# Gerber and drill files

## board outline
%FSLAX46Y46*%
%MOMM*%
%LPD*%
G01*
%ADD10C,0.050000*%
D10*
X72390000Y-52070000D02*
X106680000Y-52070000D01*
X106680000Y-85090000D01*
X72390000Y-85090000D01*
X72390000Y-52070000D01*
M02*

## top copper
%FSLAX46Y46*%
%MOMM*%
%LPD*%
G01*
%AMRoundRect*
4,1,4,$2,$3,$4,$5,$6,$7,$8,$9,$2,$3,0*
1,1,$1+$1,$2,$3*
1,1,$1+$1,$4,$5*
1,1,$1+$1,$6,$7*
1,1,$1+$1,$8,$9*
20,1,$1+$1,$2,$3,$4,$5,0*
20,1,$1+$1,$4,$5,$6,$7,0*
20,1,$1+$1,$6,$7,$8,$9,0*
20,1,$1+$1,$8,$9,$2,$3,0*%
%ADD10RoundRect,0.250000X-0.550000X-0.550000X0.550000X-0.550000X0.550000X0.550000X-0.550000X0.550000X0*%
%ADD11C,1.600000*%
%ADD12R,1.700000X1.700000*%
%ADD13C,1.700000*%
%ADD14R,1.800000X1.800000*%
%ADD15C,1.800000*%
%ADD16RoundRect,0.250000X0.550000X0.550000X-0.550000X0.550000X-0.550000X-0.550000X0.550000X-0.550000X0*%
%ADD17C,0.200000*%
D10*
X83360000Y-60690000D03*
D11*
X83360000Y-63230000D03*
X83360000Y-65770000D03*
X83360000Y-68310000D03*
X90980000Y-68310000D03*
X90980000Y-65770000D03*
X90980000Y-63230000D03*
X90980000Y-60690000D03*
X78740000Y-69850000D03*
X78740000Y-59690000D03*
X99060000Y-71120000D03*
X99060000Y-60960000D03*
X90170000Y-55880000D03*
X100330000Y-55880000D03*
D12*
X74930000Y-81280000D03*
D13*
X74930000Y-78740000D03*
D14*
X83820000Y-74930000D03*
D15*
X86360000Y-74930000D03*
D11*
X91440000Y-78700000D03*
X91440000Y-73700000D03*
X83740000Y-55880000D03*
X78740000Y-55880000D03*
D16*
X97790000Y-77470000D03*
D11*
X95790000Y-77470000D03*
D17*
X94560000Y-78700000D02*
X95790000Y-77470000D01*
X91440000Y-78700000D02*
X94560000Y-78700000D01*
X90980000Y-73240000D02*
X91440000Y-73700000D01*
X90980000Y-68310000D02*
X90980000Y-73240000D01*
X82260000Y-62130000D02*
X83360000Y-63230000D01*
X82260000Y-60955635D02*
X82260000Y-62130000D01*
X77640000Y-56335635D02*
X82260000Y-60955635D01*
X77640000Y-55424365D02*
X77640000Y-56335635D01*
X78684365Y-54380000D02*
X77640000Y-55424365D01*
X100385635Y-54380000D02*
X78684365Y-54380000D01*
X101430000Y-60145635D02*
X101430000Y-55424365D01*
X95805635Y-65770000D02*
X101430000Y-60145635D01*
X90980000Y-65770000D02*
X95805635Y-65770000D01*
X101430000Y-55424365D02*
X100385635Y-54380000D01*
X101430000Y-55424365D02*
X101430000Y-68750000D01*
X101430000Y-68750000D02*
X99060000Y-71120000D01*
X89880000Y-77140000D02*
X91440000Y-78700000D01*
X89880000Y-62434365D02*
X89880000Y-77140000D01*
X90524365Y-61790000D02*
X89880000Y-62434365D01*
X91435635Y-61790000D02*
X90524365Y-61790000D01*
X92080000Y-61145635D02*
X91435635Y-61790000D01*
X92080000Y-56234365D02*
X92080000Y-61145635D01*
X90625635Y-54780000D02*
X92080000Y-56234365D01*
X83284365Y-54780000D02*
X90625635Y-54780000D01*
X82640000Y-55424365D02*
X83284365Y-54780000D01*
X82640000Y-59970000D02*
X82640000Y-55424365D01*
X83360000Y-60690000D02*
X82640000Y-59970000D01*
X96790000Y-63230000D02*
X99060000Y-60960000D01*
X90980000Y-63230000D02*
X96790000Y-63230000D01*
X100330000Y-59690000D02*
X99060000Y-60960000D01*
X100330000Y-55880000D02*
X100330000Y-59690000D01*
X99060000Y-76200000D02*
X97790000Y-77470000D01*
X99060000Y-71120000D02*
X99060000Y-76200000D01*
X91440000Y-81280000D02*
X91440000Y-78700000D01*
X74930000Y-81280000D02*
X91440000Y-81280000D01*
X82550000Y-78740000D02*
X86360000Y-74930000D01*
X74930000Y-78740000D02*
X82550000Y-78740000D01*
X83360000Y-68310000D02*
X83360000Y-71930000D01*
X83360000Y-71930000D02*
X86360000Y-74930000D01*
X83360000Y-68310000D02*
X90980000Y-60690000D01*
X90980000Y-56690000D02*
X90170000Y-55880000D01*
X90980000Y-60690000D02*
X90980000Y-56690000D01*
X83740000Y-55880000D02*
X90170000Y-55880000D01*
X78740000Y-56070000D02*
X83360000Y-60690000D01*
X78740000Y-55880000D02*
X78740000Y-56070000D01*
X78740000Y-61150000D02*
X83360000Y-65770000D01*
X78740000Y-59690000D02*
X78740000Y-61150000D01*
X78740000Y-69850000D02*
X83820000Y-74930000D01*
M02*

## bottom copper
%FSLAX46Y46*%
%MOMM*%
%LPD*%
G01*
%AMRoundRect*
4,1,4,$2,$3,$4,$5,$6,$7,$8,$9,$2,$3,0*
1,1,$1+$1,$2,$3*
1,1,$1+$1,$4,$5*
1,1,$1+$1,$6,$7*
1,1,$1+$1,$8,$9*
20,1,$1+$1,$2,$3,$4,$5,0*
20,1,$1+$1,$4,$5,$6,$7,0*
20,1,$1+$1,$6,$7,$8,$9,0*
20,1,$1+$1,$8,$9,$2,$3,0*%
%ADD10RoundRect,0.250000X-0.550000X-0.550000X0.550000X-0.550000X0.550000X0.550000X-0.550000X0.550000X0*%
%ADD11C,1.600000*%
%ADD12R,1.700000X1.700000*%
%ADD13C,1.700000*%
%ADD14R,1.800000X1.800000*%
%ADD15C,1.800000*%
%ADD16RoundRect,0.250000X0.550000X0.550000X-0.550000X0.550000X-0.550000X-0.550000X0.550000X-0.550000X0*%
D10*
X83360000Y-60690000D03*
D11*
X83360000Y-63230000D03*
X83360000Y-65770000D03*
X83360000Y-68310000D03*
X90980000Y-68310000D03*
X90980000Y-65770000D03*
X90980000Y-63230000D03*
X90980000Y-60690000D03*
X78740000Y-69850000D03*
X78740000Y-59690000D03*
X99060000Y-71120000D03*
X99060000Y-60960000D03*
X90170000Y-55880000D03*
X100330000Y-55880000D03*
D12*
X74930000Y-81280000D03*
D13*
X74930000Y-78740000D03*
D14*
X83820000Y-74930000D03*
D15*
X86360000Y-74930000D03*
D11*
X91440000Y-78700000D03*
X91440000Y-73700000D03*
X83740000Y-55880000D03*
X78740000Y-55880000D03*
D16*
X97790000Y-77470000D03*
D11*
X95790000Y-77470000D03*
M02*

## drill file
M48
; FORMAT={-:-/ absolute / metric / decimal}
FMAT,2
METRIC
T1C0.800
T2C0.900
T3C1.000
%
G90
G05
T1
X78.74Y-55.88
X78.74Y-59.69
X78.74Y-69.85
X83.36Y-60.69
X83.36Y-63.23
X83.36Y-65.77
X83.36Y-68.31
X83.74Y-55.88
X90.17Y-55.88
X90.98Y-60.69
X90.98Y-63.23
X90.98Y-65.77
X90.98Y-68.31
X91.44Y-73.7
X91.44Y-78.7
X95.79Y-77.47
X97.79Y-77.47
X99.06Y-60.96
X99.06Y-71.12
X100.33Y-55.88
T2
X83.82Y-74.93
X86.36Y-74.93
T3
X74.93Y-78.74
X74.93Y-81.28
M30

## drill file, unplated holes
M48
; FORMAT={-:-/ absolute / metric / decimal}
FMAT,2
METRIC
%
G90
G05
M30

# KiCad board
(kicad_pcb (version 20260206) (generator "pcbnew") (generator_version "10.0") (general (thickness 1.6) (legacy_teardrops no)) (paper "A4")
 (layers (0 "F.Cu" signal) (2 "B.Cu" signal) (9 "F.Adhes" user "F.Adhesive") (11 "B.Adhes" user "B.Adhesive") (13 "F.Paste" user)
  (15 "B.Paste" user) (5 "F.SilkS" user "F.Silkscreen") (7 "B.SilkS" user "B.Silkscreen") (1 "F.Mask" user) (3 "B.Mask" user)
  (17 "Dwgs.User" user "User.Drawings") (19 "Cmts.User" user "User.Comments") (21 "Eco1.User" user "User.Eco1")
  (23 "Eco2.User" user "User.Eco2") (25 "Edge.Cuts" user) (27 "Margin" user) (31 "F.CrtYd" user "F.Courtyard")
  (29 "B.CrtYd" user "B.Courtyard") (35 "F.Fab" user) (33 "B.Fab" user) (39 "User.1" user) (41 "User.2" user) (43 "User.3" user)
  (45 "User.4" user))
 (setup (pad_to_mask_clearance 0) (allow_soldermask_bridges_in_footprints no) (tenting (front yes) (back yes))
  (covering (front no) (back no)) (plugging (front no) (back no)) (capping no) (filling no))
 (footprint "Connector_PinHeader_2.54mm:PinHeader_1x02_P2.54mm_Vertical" (layer "F.Cu") (at 74.93 81.28 180)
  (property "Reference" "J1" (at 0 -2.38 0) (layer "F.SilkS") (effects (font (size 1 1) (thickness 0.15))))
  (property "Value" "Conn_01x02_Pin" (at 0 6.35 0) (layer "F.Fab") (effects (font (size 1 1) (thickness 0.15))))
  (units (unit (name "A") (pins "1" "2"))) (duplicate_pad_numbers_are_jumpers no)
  (pad "1" thru_hole rect (at 0 0 180) (size 1.7 1.7) (drill 1) (layers "*.Cu" "*.Mask") (remove_unused_layers no) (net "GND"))
  (pad "2" thru_hole circle (at 0 2.54 180) (size 1.7 1.7) (drill 1) (layers "*.Cu" "*.Mask") (remove_unused_layers no) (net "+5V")))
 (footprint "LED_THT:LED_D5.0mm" (layer "F.Cu") (at 83.82 74.93)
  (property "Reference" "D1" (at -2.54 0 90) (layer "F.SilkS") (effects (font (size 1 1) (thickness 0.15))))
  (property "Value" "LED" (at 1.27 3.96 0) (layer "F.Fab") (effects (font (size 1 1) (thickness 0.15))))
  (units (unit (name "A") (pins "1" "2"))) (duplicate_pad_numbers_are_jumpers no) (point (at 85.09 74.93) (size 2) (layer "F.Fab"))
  (pad "1" thru_hole rect (at 0 0) (size 1.8 1.8) (drill 0.9) (layers "*.Cu" "*.Mask") (remove_unused_layers no) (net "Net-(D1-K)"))
  (pad "2" thru_hole circle (at 2.54 0) (size 1.8 1.8) (drill 0.9) (layers "*.Cu" "*.Mask") (remove_unused_layers no) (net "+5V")))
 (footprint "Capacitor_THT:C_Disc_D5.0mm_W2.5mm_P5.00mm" (layer "F.Cu") (at 78.74 55.88)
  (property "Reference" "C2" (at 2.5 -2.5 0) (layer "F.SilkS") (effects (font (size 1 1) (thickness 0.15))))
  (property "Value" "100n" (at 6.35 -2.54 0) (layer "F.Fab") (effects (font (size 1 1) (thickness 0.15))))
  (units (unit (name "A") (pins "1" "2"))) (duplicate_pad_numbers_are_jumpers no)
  (pad "1" thru_hole circle (at 0 0) (size 1.6 1.6) (drill 0.8) (layers "*.Cu" "*.Mask") (remove_unused_layers no) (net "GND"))
  (pad "2" thru_hole circle (at 5 0) (size 1.6 1.6) (drill 0.8) (layers "*.Cu" "*.Mask") (remove_unused_layers no) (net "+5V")))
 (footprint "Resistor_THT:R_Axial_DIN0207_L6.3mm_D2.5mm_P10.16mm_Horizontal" (layer "F.Cu") (at 100.33 55.88 180)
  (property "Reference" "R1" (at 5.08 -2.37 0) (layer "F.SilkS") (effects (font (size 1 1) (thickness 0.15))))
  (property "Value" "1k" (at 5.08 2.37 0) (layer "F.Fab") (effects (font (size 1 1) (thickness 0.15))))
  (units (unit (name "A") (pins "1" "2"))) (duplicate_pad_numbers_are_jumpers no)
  (pad "1" thru_hole circle (at 0 0 180) (size 1.6 1.6) (drill 0.8) (layers "*.Cu" "*.Mask") (remove_unused_layers no)
   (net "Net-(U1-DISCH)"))
  (pad "2" thru_hole circle (at 10.16 0 180) (size 1.6 1.6) (drill 0.8) (layers "*.Cu" "*.Mask") (remove_unused_layers no) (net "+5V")))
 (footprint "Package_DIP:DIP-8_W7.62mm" (layer "F.Cu") (at 83.36 60.69)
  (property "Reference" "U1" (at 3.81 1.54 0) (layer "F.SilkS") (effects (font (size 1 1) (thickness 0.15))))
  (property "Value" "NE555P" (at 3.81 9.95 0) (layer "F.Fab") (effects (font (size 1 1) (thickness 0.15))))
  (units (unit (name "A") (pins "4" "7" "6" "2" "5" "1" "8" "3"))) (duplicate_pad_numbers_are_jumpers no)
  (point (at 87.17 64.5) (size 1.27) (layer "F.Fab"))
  (pad "1" thru_hole roundrect (at 0 0) (size 1.6 1.6) (drill 0.8) (layers "*.Cu" "*.Mask") (remove_unused_layers no)
   (roundrect_rratio 0.15625) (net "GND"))
  (pad "2" thru_hole circle (at 0 2.54) (size 1.6 1.6) (drill 0.8) (layers "*.Cu" "*.Mask") (remove_unused_layers no) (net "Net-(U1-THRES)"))
  (pad "3" thru_hole circle (at 0 5.08) (size 1.6 1.6) (drill 0.8) (layers "*.Cu" "*.Mask") (remove_unused_layers no) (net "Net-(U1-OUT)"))
  (pad "4" thru_hole circle (at 0 7.62) (size 1.6 1.6) (drill 0.8) (layers "*.Cu" "*.Mask") (remove_unused_layers no) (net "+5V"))
  (pad "5" thru_hole circle (at 7.62 7.62) (size 1.6 1.6) (drill 0.8) (layers "*.Cu" "*.Mask") (remove_unused_layers no)
   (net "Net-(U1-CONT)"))
  (pad "6" thru_hole circle (at 7.62 5.08) (size 1.6 1.6) (drill 0.8) (layers "*.Cu" "*.Mask") (remove_unused_layers no)
   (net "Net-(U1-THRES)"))
  (pad "7" thru_hole circle (at 7.62 2.54) (size 1.6 1.6) (drill 0.8) (layers "*.Cu" "*.Mask") (remove_unused_layers no)
   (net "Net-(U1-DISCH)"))
  (pad "8" thru_hole circle (at 7.62 0) (size 1.6 1.6) (drill 0.8) (layers "*.Cu" "*.Mask") (remove_unused_layers no) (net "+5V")))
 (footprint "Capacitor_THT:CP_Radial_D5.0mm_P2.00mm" (layer "F.Cu") (at 97.79 77.47 180)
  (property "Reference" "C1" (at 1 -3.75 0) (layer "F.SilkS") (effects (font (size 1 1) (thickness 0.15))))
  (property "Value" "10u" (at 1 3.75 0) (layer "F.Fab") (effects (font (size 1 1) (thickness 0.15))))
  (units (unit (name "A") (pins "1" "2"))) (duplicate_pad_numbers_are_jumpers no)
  (pad "1" thru_hole roundrect (at 0 0 180) (size 1.6 1.6) (drill 0.8) (layers "*.Cu" "*.Mask") (remove_unused_layers no)
   (roundrect_rratio 0.15625) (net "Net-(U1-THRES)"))
  (pad "2" thru_hole circle (at 2 0 180) (size 1.6 1.6) (drill 0.8) (layers "*.Cu" "*.Mask") (remove_unused_layers no) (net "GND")))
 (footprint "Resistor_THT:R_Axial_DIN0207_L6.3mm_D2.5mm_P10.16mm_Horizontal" (layer "F.Cu") (at 99.06 60.96 -90)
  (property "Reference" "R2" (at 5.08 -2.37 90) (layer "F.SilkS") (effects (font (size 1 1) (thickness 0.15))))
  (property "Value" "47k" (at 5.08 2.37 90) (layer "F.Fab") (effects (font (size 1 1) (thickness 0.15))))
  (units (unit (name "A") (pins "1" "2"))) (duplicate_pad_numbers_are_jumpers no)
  (pad "1" thru_hole circle (at 0 0 270) (size 1.6 1.6) (drill 0.8) (layers "*.Cu" "*.Mask") (remove_unused_layers no)
   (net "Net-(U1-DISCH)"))
  (pad "2" thru_hole circle (at 10.16 0 270) (size 1.6 1.6) (drill 0.8) (layers "*.Cu" "*.Mask") (remove_unused_layers no)
   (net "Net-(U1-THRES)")))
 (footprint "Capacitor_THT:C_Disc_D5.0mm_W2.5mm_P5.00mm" (layer "F.Cu") (at 91.44 78.7 90)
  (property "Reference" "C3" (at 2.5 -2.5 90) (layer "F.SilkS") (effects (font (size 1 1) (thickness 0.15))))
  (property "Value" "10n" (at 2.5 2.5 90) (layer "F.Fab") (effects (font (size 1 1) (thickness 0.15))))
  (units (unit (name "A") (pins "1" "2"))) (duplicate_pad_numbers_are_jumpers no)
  (pad "1" thru_hole circle (at 0 0 90) (size 1.6 1.6) (drill 0.8) (layers "*.Cu" "*.Mask") (remove_unused_layers no) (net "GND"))
  (pad "2" thru_hole circle (at 5 0 90) (size 1.6 1.6) (drill 0.8) (layers "*.Cu" "*.Mask") (remove_unused_layers no) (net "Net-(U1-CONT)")))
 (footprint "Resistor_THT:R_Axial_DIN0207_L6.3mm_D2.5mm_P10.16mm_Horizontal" (layer "F.Cu") (at 78.74 59.69 -90)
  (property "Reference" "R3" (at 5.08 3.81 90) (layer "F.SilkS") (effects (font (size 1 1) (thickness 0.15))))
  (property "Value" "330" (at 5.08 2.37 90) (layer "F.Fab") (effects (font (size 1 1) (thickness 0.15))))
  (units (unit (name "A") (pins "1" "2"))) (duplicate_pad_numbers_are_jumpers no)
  (pad "1" thru_hole circle (at 0 0 270) (size 1.6 1.6) (drill 0.8) (layers "*.Cu" "*.Mask") (remove_unused_layers no) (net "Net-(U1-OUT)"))
  (pad "2" thru_hole circle (at 10.16 0 270) (size 1.6 1.6) (drill 0.8) (layers "*.Cu" "*.Mask") (remove_unused_layers no)
   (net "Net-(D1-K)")))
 (gr_rect (start 72.39 52.07) (end 106.68 85.09) (stroke (width 0.05) (type default)) (fill no) (layer "Edge.Cuts"))
 (segment (start 91.44 78.7) (end 94.56 78.7) (width 0.2) (layer "F.Cu") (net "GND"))
 (segment (start 78.74 55.88) (end 78.74 56.07) (width 0.2) (layer "F.Cu") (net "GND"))
 (segment (start 78.74 56.07) (end 83.36 60.69) (width 0.2) (layer "F.Cu") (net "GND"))
 (segment (start 82.64 55.424365) (end 83.284365 54.78) (width 0.2) (layer "F.Cu") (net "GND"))
 (segment (start 90.625635 54.78) (end 92.08 56.234365) (width 0.2) (layer "F.Cu") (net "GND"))
 (segment (start 92.08 61.145635) (end 91.435635 61.79) (width 0.2) (layer "F.Cu") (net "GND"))
 (segment (start 91.435635 61.79) (end 90.524365 61.79) (width 0.2) (layer "F.Cu") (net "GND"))
 (segment (start 89.88 77.14) (end 91.44 78.7) (width 0.2) (layer "F.Cu") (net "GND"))
 (segment (start 94.56 78.7) (end 95.79 77.47) (width 0.2) (layer "F.Cu") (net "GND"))
 (segment (start 83.36 60.69) (end 82.64 59.97) (width 0.2) (layer "F.Cu") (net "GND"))
 (segment (start 91.44 81.28) (end 91.44 78.7) (width 0.2) (layer "F.Cu") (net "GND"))
 (segment (start 74.93 81.28) (end 91.44 81.28) (width 0.2) (layer "F.Cu") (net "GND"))
 (segment (start 89.88 62.434365) (end 89.88 77.14) (width 0.2) (layer "F.Cu") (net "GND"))
 (segment (start 90.524365 61.79) (end 89.88 62.434365) (width 0.2) (layer "F.Cu") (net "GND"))
 (segment (start 82.64 59.97) (end 82.64 55.424365) (width 0.2) (layer "F.Cu") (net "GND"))
 (segment (start 92.08 56.234365) (end 92.08 61.145635) (width 0.2) (layer "F.Cu") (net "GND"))
 (segment (start 83.284365 54.78) (end 90.625635 54.78) (width 0.2) (layer "F.Cu") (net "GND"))
 (segment (start 83.36 71.93) (end 86.36 74.93) (width 0.2) (layer "F.Cu") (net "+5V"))
 (segment (start 90.98 60.69) (end 90.98 56.69) (width 0.2) (layer "F.Cu") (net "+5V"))
 (segment (start 83.74 55.88) (end 90.17 55.88) (width 0.2) (layer "F.Cu") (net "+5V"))
 (segment (start 82.55 78.74) (end 86.36 74.93) (width 0.2) (layer "F.Cu") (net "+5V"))
 (segment (start 90.98 56.69) (end 90.17 55.88) (width 0.2) (layer "F.Cu") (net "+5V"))
 (segment (start 83.36 68.31) (end 90.98 60.69) (width 0.2) (layer "F.Cu") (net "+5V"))
 (segment (start 83.36 68.31) (end 83.36 71.93) (width 0.2) (layer "F.Cu") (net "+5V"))
 (segment (start 74.93 78.74) (end 82.55 78.74) (width 0.2) (layer "F.Cu") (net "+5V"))
 (segment (start 100.33 55.88) (end 100.33 59.69) (width 0.2) (layer "F.Cu") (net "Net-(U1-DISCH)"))
 (segment (start 100.33 59.69) (end 99.06 60.96) (width 0.2) (layer "F.Cu") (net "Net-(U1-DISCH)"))
 (segment (start 90.98 63.23) (end 96.79 63.23) (width 0.2) (layer "F.Cu") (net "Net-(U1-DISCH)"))
 (segment (start 96.79 63.23) (end 99.06 60.96) (width 0.2) (layer "F.Cu") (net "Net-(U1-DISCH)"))
 (segment (start 78.74 61.15) (end 83.36 65.77) (width 0.2) (layer "F.Cu") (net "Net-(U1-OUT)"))
 (segment (start 78.74 59.69) (end 78.74 61.15) (width 0.2) (layer "F.Cu") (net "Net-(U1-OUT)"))
 (segment (start 101.43 60.145635) (end 101.43 55.424365) (width 0.2) (layer "F.Cu") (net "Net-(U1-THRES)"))
 (segment (start 90.98 65.77) (end 95.805635 65.77) (width 0.2) (layer "F.Cu") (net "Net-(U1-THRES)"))
 (segment (start 95.805635 65.77) (end 101.43 60.145635) (width 0.2) (layer "F.Cu") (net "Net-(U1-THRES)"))
 (segment (start 99.06 71.12) (end 99.06 76.2) (width 0.2) (layer "F.Cu") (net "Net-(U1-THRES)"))
 (segment (start 101.43 55.424365) (end 100.385635 54.38) (width 0.2) (layer "F.Cu") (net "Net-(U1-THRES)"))
 (segment (start 77.64 56.335635) (end 82.26 60.955635) (width 0.2) (layer "F.Cu") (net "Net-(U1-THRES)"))
 (segment (start 82.26 60.955635) (end 82.26 62.13) (width 0.2) (layer "F.Cu") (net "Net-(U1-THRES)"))
 (segment (start 78.684365 54.38) (end 77.64 55.424365) (width 0.2) (layer "F.Cu") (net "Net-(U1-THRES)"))
 (segment (start 82.26 62.13) (end 83.36 63.23) (width 0.2) (layer "F.Cu") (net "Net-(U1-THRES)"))
 (segment (start 101.43 68.75) (end 99.06 71.12) (width 0.2) (layer "F.Cu") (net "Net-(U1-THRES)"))
 (segment (start 99.06 76.2) (end 97.79 77.47) (width 0.2) (layer "F.Cu") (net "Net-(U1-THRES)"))
 (segment (start 101.43 55.424365) (end 101.43 68.75) (width 0.2) (layer "F.Cu") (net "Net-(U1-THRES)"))
 (segment (start 100.385635 54.38) (end 78.684365 54.38) (width 0.2) (layer "F.Cu") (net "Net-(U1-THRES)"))
 (segment (start 77.64 55.424365) (end 77.64 56.335635) (width 0.2) (layer "F.Cu") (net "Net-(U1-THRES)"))
 (segment (start 90.98 73.24) (end 91.44 73.7) (width 0.2) (layer "F.Cu") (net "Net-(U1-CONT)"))
 (segment (start 90.98 68.31) (end 90.98 73.24) (width 0.2) (layer "F.Cu") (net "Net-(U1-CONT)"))
 (segment (start 78.74 69.85) (end 83.82 74.93) (width 0.2) (layer "F.Cu") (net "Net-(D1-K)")))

